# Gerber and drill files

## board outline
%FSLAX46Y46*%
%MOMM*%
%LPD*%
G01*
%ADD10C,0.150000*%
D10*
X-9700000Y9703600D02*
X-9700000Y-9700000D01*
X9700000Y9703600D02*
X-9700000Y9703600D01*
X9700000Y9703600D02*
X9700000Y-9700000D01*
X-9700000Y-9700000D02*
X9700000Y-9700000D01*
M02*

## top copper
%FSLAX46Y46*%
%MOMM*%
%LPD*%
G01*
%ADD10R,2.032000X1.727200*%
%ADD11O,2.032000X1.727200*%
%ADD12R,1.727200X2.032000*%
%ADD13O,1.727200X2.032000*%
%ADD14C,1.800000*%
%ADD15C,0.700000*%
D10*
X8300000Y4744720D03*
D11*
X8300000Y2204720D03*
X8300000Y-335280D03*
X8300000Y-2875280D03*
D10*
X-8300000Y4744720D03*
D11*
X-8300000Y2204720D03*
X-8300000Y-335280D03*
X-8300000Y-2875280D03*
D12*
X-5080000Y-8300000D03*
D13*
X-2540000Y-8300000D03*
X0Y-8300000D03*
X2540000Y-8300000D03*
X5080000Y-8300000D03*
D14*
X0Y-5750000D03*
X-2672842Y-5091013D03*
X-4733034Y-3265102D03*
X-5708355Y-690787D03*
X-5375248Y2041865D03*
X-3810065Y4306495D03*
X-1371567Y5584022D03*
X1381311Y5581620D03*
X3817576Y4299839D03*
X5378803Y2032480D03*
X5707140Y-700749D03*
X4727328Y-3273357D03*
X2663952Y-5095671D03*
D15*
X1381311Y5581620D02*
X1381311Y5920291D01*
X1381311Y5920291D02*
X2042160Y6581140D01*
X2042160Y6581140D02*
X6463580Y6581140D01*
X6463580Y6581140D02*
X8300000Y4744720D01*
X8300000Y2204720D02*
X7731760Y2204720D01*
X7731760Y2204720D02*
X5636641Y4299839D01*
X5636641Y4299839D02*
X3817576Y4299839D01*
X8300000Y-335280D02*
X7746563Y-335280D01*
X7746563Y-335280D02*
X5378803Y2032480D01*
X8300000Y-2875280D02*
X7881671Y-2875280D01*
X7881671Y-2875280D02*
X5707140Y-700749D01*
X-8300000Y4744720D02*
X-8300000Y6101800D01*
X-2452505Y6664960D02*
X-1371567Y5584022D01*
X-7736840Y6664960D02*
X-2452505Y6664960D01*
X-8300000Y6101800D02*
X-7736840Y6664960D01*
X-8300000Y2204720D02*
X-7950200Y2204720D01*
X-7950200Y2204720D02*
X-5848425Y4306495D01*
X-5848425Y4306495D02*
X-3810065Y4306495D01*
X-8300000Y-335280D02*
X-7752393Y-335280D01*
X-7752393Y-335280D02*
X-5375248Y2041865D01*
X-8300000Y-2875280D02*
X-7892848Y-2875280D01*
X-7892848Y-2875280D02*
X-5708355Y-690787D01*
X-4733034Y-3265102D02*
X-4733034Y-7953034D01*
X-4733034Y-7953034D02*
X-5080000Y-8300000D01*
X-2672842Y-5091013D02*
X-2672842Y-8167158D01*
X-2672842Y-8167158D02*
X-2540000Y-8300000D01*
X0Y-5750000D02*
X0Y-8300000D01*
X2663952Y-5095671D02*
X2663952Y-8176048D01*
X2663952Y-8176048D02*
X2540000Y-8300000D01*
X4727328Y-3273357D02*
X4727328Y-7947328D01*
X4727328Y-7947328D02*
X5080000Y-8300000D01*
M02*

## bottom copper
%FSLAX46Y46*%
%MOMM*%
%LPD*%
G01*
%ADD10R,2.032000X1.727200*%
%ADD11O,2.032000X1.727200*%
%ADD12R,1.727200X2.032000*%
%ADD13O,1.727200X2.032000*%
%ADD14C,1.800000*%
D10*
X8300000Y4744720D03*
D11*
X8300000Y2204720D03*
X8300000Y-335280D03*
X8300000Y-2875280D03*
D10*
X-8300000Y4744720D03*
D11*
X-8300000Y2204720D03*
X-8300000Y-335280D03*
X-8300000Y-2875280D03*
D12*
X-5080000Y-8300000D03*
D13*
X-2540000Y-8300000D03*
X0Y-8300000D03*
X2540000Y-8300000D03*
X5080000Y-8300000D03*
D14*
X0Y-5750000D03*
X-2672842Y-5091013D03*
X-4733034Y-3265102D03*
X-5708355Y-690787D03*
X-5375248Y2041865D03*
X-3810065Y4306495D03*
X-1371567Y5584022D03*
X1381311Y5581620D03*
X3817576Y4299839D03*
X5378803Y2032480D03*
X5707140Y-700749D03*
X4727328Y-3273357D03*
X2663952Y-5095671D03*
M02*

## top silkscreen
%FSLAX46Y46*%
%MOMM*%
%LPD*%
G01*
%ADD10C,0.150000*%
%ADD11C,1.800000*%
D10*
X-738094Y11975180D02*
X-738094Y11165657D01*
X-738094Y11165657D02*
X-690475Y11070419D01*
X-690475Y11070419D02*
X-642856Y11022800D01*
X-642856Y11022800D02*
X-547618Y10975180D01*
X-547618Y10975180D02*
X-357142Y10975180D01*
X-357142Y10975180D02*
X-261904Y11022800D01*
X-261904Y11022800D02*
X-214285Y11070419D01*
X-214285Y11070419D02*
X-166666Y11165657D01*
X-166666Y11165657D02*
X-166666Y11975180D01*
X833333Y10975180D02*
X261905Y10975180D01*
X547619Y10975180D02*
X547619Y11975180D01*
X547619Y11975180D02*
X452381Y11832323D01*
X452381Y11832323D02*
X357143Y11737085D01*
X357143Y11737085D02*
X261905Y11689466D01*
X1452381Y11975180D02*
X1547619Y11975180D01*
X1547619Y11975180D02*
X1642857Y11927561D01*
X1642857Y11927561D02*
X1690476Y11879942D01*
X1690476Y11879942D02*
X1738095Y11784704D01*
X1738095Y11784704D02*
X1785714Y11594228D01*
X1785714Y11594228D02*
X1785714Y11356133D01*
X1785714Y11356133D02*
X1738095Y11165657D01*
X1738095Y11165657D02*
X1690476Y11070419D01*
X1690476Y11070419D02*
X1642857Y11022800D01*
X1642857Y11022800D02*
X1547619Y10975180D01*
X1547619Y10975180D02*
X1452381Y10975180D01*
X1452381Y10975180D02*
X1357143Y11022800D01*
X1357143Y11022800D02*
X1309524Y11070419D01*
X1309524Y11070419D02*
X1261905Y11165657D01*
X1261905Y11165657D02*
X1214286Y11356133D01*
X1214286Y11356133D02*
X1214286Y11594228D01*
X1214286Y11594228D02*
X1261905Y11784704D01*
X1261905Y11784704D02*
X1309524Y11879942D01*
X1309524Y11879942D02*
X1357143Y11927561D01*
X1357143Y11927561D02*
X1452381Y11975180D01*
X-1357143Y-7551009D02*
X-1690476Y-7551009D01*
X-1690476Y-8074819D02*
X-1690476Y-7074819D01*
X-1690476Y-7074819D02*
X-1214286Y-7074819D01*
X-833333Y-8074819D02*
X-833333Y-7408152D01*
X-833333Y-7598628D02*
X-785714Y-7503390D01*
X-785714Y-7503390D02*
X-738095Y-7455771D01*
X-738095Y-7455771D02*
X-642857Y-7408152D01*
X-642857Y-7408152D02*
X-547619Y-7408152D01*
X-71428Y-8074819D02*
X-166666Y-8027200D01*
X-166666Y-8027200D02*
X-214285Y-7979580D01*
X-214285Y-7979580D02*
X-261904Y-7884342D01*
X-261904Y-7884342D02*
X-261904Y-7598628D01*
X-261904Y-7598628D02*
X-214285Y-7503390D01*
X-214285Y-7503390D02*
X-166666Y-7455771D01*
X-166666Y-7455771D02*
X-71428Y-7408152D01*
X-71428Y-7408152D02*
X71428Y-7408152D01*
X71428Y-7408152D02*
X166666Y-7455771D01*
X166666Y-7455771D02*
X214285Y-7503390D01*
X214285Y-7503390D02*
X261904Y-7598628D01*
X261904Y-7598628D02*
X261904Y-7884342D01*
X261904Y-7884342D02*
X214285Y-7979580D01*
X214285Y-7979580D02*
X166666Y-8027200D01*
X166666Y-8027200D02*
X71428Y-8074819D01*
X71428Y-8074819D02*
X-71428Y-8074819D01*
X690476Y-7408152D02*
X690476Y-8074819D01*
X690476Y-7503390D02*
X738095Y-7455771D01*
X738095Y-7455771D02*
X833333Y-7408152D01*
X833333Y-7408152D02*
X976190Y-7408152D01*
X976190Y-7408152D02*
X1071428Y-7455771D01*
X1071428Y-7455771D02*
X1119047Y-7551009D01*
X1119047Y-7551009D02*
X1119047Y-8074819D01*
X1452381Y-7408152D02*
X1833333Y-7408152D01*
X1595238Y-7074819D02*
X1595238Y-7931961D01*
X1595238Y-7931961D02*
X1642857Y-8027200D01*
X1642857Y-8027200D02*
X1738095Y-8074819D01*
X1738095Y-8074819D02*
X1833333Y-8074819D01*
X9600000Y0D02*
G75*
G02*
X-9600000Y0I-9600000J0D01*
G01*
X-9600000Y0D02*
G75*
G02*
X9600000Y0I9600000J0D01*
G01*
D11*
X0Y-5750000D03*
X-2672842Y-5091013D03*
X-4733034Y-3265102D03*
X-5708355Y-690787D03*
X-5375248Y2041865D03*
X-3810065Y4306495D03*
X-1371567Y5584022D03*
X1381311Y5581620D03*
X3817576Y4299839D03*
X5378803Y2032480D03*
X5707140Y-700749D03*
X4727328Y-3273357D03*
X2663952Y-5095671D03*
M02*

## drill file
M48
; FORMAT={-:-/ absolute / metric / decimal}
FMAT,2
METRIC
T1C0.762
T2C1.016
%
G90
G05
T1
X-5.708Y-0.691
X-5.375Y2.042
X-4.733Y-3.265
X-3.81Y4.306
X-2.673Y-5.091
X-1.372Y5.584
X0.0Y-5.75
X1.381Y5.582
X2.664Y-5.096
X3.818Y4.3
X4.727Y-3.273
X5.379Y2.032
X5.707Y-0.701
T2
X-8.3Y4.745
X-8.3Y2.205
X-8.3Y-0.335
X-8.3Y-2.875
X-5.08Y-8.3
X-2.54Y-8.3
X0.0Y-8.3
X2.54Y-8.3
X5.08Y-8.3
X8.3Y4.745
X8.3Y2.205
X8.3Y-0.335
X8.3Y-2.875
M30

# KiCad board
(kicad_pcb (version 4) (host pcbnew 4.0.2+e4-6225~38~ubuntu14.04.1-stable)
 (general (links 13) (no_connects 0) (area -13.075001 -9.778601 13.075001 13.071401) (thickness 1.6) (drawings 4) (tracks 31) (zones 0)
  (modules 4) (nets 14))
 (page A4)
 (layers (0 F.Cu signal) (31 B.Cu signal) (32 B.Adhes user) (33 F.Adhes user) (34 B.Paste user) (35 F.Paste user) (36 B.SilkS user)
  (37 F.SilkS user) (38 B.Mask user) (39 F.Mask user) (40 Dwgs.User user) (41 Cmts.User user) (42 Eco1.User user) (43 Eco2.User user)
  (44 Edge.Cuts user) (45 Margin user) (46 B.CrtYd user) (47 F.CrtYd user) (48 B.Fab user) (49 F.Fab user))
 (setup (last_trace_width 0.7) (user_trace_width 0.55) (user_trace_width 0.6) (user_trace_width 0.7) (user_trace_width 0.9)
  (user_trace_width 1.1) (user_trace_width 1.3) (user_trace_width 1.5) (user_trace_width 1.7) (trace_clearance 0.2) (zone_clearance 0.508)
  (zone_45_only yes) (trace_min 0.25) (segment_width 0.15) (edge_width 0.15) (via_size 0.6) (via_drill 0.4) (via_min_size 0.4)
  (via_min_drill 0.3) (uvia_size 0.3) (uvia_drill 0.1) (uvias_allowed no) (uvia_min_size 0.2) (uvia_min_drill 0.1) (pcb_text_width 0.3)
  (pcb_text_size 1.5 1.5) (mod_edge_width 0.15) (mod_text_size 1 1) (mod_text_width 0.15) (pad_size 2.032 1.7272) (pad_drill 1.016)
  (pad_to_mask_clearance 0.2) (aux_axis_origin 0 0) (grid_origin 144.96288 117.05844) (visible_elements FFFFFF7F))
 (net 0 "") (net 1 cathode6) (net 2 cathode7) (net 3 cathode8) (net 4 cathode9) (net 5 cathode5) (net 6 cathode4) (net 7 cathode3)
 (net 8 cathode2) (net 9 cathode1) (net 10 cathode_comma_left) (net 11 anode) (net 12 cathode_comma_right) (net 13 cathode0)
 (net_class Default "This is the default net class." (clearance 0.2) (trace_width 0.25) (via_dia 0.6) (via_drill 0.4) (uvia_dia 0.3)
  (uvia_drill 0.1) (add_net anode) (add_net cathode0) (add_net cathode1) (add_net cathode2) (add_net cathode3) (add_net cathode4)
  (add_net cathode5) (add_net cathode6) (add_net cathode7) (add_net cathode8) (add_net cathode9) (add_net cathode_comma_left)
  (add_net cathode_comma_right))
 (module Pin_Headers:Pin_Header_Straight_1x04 (layer B.Cu) (at 8.3 -4.74472 180)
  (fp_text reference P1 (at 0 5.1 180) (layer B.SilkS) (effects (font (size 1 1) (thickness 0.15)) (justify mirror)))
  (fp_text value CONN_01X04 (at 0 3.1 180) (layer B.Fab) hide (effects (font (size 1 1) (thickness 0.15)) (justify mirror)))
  (pad 1 thru_hole rect (at 0 0 180) (size 2.032 1.7272) (drill 1.016) (layers *.Cu *.Mask B.SilkS) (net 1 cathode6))
  (pad 2 thru_hole oval (at 0 -2.54 180) (size 2.032 1.7272) (drill 1.016) (layers *.Cu *.Mask B.SilkS) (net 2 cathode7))
  (pad 3 thru_hole oval (at 0 -5.08 180) (size 2.032 1.7272) (drill 1.016) (layers *.Cu *.Mask B.SilkS) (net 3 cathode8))
  (pad 4 thru_hole oval (at 0 -7.62 180) (size 2.032 1.7272) (drill 1.016) (layers *.Cu *.Mask B.SilkS) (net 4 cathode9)))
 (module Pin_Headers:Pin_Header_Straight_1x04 (layer B.Cu) (at -8.3 -4.74472 180)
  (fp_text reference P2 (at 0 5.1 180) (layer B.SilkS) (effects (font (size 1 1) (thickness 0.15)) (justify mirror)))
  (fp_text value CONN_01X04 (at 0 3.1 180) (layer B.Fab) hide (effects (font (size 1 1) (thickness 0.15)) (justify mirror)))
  (pad 1 thru_hole rect (at 0 0 180) (size 2.032 1.7272) (drill 1.016) (layers *.Cu *.Mask B.SilkS) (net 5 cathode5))
  (pad 2 thru_hole oval (at 0 -2.54 180) (size 2.032 1.7272) (drill 1.016) (layers *.Cu *.Mask B.SilkS) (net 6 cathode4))
  (pad 3 thru_hole oval (at 0 -5.08 180) (size 2.032 1.7272) (drill 1.016) (layers *.Cu *.Mask B.SilkS) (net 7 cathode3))
  (pad 4 thru_hole oval (at 0 -7.62 180) (size 2.032 1.7272) (drill 1.016) (layers *.Cu *.Mask B.SilkS) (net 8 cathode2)))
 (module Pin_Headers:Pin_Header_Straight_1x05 (layer B.Cu) (at -5.08 8.3 270)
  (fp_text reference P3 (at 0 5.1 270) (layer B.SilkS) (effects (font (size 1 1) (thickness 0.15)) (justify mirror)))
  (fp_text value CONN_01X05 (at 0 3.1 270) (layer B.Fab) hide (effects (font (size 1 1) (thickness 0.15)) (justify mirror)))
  (pad 1 thru_hole rect (at 0 0 270) (size 2.032 1.7272) (drill 1.016) (layers *.Cu *.Mask B.SilkS) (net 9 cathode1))
  (pad 2 thru_hole oval (at 0 -2.54 270) (size 2.032 1.7272) (drill 1.016) (layers *.Cu *.Mask B.SilkS) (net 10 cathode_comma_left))
  (pad 3 thru_hole oval (at 0 -5.08 270) (size 2.032 1.7272) (drill 1.016) (layers *.Cu *.Mask B.SilkS) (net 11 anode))
  (pad 4 thru_hole oval (at 0 -7.62 270) (size 2.032 1.7272) (drill 1.016) (layers *.Cu *.Mask B.SilkS) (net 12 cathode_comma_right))
  (pad 5 thru_hole oval (at 0 -10.16 270) (size 2.032 1.7272) (drill 1.016) (layers *.Cu *.Mask B.SilkS) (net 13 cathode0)))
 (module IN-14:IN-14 (layer F.Cu) (at 0 0)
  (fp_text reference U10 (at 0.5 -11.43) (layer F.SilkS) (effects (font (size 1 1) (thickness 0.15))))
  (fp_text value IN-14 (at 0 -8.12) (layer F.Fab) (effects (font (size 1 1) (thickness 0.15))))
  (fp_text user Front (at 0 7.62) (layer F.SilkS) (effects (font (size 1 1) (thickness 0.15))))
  (fp_circle (center 0 0) (end 0 9.6) (layer F.SilkS) (width 0.15))
  (pad 1 thru_hole circle (at 0 5.75) (size 1.8 1.8) (drill 0.762) (layers *.Cu *.Mask F.SilkS) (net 11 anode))
  (pad 2 thru_hole circle (at -2.672842 5.091013) (size 1.8 1.8) (drill 0.762) (layers *.Cu *.Mask F.SilkS) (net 10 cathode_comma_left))
  (pad 3 thru_hole circle (at -4.733034 3.265102) (size 1.8 1.8) (drill 0.762) (layers *.Cu *.Mask F.SilkS) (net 9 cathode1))
  (pad 4 thru_hole circle (at -5.708355 0.690787) (size 1.8 1.8) (drill 0.762) (layers *.Cu *.Mask F.SilkS) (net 8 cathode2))
  (pad 5 thru_hole circle (at -5.375248 -2.041865) (size 1.8 1.8) (drill 0.762) (layers *.Cu *.Mask F.SilkS) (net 7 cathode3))
  (pad 6 thru_hole circle (at -3.810065 -4.306495) (size 1.8 1.8) (drill 0.762) (layers *.Cu *.Mask F.SilkS) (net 6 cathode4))
  (pad 7 thru_hole circle (at -1.371567 -5.584022) (size 1.8 1.8) (drill 0.762) (layers *.Cu *.Mask F.SilkS) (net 5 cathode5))
  (pad 8 thru_hole circle (at 1.381311 -5.58162) (size 1.8 1.8) (drill 0.762) (layers *.Cu *.Mask F.SilkS) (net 1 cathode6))
  (pad 9 thru_hole circle (at 3.817576 -4.299839) (size 1.8 1.8) (drill 0.762) (layers *.Cu *.Mask F.SilkS) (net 2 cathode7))
  (pad 10 thru_hole circle (at 5.378803 -2.03248) (size 1.8 1.8) (drill 0.762) (layers *.Cu *.Mask F.SilkS) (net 3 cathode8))
  (pad 11 thru_hole circle (at 5.70714 0.700749) (size 1.8 1.8) (drill 0.762) (layers *.Cu *.Mask F.SilkS) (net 4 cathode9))
  (pad 12 thru_hole circle (at 4.727328 3.273357) (size 1.8 1.8) (drill 0.762) (layers *.Cu *.Mask F.SilkS) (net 13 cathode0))
  (pad 13 thru_hole circle (at 2.663952 5.095671) (size 1.8 1.8) (drill 0.762) (layers *.Cu *.Mask F.SilkS) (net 12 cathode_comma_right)))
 (gr_line (start -9.7 -9.7036) (end -9.7 9.7) (angle 90) (layer Edge.Cuts) (width 0.15))
 (gr_line (start 9.7 -9.7036) (end -9.7 -9.7036) (angle 90) (layer Edge.Cuts) (width 0.15))
 (gr_line (start 9.7 -9.7036) (end 9.7 9.7) (angle 90) (layer Edge.Cuts) (width 0.15))
 (gr_line (start -9.7 9.7) (end 9.7 9.7) (angle 90) (layer Edge.Cuts) (width 0.15))
 (segment (start 1.381311 -5.58162) (end 1.381311 -5.920291) (width 0.7) (layer F.Cu) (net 1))
 (segment (start 1.381311 -5.920291) (end 2.04216 -6.58114) (width 0.7) (layer F.Cu) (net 1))
 (segment (start 2.04216 -6.58114) (end 6.46358 -6.58114) (width 0.7) (layer F.Cu) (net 1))
 (segment (start 6.46358 -6.58114) (end 8.3 -4.74472) (width 0.7) (layer F.Cu) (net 1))
 (segment (start 8.3 -2.20472) (end 7.73176 -2.20472) (width 0.7) (layer F.Cu) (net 2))
 (segment (start 7.73176 -2.20472) (end 5.636641 -4.299839) (width 0.7) (layer F.Cu) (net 2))
 (segment (start 5.636641 -4.299839) (end 3.817576 -4.299839) (width 0.7) (layer F.Cu) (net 2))
 (segment (start 8.3 0.33528) (end 7.746563 0.33528) (width 0.7) (layer F.Cu) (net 3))
 (segment (start 7.746563 0.33528) (end 5.378803 -2.03248) (width 0.7) (layer F.Cu) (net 3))
 (segment (start 8.3 2.87528) (end 7.881671 2.87528) (width 0.7) (layer F.Cu) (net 4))
 (segment (start 7.881671 2.87528) (end 5.70714 0.700749) (width 0.7) (layer F.Cu) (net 4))
 (segment (start -8.3 -4.74472) (end -8.3 -6.1018) (width 0.7) (layer F.Cu) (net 5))
 (segment (start -2.452505 -6.66496) (end -1.371567 -5.584022) (width 0.7) (layer F.Cu) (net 5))
 (segment (start -7.73684 -6.66496) (end -2.452505 -6.66496) (width 0.7) (layer F.Cu) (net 5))
 (segment (start -8.3 -6.1018) (end -7.73684 -6.66496) (width 0.7) (layer F.Cu) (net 5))
 (segment (start -8.3 -2.20472) (end -7.9502 -2.20472) (width 0.7) (layer F.Cu) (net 6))
 (segment (start -7.9502 -2.20472) (end -5.848425 -4.306495) (width 0.7) (layer F.Cu) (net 6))
 (segment (start -5.848425 -4.306495) (end -3.810065 -4.306495) (width 0.7) (layer F.Cu) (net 6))
 (segment (start -8.3 0.33528) (end -7.752393 0.33528) (width 0.7) (layer F.Cu) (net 7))
 (segment (start -7.752393 0.33528) (end -5.375248 -2.041865) (width 0.7) (layer F.Cu) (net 7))
 (segment (start -8.3 2.87528) (end -7.892848 2.87528) (width 0.7) (layer F.Cu) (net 8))
 (segment (start -7.892848 2.87528) (end -5.708355 0.690787) (width 0.7) (layer F.Cu) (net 8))
 (segment (start -4.733034 3.265102) (end -4.733034 7.953034) (width 0.7) (layer F.Cu) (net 9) (status C00000))
 (segment (start -4.733034 7.953034) (end -5.08 8.3) (width 0.7) (layer F.Cu) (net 9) (status C00000))
 (segment (start -2.672842 5.091013) (end -2.672842 8.167158) (width 0.7) (layer F.Cu) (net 10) (status C00000))
 (segment (start -2.672842 8.167158) (end -2.54 8.3) (width 0.7) (layer F.Cu) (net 10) (status C00000))
 (segment (start 0 5.75) (end 0 8.3) (width 0.7) (layer F.Cu) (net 11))
 (segment (start 2.663952 5.095671) (end 2.663952 8.176048) (width 0.7) (layer F.Cu) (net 12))
 (segment (start 2.663952 8.176048) (end 2.54 8.3) (width 0.7) (layer F.Cu) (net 12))
 (segment (start 4.727328 3.273357) (end 4.727328 7.947328) (width 0.7) (layer F.Cu) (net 13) (status C00000))
 (segment (start 4.727328 7.947328) (end 5.08 8.3) (width 0.7) (layer F.Cu) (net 13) (status C00000)))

